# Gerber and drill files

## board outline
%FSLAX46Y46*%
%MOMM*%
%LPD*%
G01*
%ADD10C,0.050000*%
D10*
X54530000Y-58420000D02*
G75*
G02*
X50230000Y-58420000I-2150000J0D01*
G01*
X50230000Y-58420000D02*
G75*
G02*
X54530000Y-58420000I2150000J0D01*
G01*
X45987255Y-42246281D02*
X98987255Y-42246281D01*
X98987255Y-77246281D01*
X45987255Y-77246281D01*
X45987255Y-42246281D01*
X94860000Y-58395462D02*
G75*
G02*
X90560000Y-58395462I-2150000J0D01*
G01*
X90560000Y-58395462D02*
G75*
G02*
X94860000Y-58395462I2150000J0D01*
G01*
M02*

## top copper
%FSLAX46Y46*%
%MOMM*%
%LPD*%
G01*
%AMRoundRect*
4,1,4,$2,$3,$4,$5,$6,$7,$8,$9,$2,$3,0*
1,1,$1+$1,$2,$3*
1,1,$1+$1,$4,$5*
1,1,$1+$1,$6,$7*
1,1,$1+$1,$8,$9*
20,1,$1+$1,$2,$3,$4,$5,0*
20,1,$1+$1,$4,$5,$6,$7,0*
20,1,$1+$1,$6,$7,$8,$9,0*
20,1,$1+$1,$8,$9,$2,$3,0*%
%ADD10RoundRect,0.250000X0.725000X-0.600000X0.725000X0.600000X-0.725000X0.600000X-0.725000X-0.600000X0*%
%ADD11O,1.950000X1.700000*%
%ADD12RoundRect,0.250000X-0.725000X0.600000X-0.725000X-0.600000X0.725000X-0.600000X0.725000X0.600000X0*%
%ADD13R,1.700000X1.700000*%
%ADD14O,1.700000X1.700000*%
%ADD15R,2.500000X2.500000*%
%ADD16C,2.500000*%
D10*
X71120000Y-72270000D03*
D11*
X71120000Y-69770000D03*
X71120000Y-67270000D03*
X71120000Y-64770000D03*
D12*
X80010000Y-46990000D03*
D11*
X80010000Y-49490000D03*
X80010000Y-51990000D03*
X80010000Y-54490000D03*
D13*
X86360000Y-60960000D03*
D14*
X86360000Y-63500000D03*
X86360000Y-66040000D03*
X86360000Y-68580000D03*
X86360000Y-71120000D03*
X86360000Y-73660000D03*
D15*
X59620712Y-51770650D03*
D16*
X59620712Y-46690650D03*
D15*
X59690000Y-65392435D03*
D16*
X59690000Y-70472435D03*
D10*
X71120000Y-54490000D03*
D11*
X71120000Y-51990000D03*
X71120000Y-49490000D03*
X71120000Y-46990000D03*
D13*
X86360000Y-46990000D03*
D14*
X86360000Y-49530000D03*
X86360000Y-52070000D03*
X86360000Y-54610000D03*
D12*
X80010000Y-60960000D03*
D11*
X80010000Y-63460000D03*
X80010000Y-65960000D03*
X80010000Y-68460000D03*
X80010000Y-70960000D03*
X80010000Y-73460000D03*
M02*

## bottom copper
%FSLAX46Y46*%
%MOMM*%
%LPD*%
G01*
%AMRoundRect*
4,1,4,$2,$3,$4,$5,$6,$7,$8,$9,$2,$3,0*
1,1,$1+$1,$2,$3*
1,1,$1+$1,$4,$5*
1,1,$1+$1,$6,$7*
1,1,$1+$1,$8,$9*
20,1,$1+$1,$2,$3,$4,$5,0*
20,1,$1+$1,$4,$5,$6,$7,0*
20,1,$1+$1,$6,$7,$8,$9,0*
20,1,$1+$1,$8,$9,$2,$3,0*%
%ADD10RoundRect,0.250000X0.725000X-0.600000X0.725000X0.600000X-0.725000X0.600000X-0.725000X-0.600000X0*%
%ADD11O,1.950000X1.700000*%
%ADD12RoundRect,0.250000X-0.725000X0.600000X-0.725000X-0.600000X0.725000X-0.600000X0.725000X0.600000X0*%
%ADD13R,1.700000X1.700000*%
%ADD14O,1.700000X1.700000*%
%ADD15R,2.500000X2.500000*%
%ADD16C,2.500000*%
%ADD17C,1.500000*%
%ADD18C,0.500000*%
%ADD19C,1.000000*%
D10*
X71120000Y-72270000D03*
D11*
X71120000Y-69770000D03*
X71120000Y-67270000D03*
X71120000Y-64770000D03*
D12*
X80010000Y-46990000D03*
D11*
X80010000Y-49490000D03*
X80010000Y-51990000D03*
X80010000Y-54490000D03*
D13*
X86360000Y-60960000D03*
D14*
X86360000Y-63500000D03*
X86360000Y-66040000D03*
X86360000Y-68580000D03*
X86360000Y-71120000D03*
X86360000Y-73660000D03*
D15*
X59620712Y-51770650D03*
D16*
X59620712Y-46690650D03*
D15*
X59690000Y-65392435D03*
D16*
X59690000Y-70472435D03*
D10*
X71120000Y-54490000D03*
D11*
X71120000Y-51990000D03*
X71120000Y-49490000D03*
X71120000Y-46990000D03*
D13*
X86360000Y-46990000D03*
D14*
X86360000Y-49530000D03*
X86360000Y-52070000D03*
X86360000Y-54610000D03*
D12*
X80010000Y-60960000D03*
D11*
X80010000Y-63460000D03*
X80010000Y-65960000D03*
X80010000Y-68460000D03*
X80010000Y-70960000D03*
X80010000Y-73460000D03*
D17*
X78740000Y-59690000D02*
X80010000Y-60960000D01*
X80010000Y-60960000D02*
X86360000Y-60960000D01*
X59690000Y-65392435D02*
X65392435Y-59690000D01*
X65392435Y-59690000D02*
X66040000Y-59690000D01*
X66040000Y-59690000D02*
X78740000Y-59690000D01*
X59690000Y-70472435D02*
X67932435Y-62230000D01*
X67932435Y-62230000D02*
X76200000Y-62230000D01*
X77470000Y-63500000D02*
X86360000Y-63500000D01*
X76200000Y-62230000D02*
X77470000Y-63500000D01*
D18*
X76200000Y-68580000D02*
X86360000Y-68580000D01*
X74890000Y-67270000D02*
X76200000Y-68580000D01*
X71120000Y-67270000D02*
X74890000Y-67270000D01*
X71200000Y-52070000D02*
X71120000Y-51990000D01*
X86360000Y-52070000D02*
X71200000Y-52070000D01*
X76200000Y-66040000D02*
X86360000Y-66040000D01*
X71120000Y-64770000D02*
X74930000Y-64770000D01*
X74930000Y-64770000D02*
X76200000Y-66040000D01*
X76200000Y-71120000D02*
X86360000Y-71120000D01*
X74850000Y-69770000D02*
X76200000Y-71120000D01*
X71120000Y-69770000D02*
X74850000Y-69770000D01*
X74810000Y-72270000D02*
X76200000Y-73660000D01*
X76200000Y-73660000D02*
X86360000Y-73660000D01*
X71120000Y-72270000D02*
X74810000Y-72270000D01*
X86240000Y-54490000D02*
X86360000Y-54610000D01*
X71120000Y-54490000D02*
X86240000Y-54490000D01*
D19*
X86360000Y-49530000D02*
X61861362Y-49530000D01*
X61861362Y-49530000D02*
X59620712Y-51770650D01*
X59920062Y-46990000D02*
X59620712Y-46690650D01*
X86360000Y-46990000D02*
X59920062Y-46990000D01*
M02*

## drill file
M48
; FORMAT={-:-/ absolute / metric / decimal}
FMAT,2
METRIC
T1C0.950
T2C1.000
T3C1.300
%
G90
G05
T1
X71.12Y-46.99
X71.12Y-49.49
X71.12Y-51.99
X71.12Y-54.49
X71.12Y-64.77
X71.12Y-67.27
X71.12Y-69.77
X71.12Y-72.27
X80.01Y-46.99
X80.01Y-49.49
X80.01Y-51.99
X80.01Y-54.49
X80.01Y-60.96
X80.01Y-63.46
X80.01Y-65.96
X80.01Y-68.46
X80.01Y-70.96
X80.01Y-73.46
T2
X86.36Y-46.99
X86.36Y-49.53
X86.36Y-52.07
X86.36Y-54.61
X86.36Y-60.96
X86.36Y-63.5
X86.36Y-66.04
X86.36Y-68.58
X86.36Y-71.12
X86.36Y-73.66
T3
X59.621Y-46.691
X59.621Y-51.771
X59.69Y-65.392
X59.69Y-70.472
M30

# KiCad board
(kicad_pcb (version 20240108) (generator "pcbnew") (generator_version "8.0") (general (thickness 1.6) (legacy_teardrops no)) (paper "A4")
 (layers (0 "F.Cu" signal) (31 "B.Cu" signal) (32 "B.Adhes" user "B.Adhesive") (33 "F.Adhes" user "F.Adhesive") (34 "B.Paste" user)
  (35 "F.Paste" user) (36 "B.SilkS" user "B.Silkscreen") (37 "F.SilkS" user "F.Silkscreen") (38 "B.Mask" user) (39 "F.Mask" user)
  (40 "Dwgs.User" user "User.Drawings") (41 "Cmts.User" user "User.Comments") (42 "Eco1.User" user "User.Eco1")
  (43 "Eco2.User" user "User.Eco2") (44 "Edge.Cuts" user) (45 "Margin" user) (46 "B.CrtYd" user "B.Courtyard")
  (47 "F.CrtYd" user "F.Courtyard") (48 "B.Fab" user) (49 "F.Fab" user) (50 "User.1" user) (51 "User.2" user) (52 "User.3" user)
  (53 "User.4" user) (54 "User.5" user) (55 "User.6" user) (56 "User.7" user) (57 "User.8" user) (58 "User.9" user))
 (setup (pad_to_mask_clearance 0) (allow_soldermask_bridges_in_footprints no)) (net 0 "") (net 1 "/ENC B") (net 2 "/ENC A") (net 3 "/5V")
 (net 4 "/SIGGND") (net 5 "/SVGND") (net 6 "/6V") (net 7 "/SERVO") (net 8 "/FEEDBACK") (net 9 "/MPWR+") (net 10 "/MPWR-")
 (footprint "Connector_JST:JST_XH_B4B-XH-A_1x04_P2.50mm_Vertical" (layer "F.Cu") (at 71.12 72.27 90)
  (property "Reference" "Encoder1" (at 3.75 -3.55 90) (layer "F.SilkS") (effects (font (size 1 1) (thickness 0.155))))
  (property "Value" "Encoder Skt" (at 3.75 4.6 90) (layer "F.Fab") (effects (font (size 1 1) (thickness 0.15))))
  (pad "1" thru_hole roundrect (at 0 0 90) (size 1.7 1.95) (drill 0.95) (layers "*.Cu" "*.Mask") (remove_unused_layers no)
   (roundrect_rratio 0.147059) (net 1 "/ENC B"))
  (pad "2" thru_hole oval (at 2.5 0 90) (size 1.7 1.95) (drill 0.95) (layers "*.Cu" "*.Mask") (remove_unused_layers no) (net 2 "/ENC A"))
  (pad "3" thru_hole oval (at 5 0 90) (size 1.7 1.95) (drill 0.95) (layers "*.Cu" "*.Mask") (remove_unused_layers no) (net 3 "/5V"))
  (pad "4" thru_hole oval (at 7.5 0 90) (size 1.7 1.95) (drill 0.95) (layers "*.Cu" "*.Mask") (remove_unused_layers no) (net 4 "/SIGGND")))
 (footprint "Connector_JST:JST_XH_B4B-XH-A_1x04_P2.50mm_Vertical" (layer "F.Cu") (at 80.01 46.99 -90)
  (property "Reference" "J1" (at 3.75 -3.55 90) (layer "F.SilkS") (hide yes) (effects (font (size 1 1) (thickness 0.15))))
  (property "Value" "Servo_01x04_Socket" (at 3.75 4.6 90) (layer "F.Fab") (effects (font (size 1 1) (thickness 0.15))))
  (pad "1" thru_hole roundrect (at 0 0 270) (size 1.7 1.95) (drill 0.95) (layers "*.Cu" "*.Mask") (remove_unused_layers no)
   (roundrect_rratio 0.147059) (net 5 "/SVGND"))
  (pad "2" thru_hole oval (at 2.5 0 270) (size 1.7 1.95) (drill 0.95) (layers "*.Cu" "*.Mask") (remove_unused_layers no) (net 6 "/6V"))
  (pad "3" thru_hole oval (at 5 0 270) (size 1.7 1.95) (drill 0.95) (layers "*.Cu" "*.Mask") (remove_unused_layers no) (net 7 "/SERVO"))
  (pad "4" thru_hole oval (at 7.5 0 270) (size 1.7 1.95) (drill 0.95) (layers "*.Cu" "*.Mask") (remove_unused_layers no) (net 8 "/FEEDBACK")))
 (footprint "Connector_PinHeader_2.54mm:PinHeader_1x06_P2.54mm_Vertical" (layer "F.Cu") (at 86.36 60.96)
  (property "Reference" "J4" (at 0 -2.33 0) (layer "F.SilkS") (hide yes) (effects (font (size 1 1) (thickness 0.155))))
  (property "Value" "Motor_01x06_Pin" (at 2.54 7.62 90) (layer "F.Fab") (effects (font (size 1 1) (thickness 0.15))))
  (pad "1" thru_hole rect (at 0 0) (size 1.7 1.7) (drill 1) (layers "*.Cu" "*.Mask") (remove_unused_layers no) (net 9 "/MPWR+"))
  (pad "2" thru_hole oval (at 0 2.54) (size 1.7 1.7) (drill 1) (layers "*.Cu" "*.Mask") (remove_unused_layers no) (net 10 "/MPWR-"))
  (pad "3" thru_hole oval (at 0 5.08) (size 1.7 1.7) (drill 1) (layers "*.Cu" "*.Mask") (remove_unused_layers no) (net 4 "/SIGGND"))
  (pad "4" thru_hole oval (at 0 7.62) (size 1.7 1.7) (drill 1) (layers "*.Cu" "*.Mask") (remove_unused_layers no) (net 3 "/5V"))
  (pad "5" thru_hole oval (at 0 10.16) (size 1.7 1.7) (drill 1) (layers "*.Cu" "*.Mask") (remove_unused_layers no) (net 2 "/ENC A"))
  (pad "6" thru_hole oval (at 0 12.7) (size 1.7 1.7) (drill 1) (layers "*.Cu" "*.Mask") (remove_unused_layers no) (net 1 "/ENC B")))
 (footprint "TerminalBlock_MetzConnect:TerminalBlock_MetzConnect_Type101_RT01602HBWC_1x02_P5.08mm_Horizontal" (layer "F.Cu")
  (at 59.620712 51.77065 90)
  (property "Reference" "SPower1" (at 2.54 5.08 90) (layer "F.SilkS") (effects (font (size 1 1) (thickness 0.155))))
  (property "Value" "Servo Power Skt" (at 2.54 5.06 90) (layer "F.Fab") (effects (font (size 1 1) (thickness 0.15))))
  (pad "1" thru_hole rect (at 0 0 90) (size 2.5 2.5) (drill 1.3) (layers "*.Cu" "*.Mask") (remove_unused_layers no) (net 6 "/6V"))
  (pad "2" thru_hole circle (at 5.08 0 90) (size 2.5 2.5) (drill 1.3) (layers "*.Cu" "*.Mask") (remove_unused_layers no) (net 5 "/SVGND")))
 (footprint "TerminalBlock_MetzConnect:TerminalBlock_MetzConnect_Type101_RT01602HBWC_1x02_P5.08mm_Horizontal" (layer "F.Cu")
  (at 59.69 65.392435 -90)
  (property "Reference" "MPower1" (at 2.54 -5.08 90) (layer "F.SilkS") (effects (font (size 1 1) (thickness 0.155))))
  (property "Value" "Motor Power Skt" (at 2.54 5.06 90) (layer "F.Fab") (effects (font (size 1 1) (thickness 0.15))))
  (pad "1" thru_hole rect (at 0 0 270) (size 2.5 2.5) (drill 1.3) (layers "*.Cu" "*.Mask") (remove_unused_layers no) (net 9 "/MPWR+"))
  (pad "2" thru_hole circle (at 5.08 0 270) (size 2.5 2.5) (drill 1.3) (layers "*.Cu" "*.Mask") (remove_unused_layers no) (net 10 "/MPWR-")))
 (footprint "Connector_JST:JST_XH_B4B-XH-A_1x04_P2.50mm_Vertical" (layer "F.Cu") (at 71.12 54.49 90)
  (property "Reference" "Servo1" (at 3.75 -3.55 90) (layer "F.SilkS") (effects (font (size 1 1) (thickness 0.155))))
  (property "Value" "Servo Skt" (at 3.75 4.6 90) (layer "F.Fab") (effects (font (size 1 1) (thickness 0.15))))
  (pad "1" thru_hole roundrect (at 0 0 90) (size 1.7 1.95) (drill 0.95) (layers "*.Cu" "*.Mask") (remove_unused_layers no)
   (roundrect_rratio 0.147059) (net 8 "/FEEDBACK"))
  (pad "2" thru_hole oval (at 2.5 0 90) (size 1.7 1.95) (drill 0.95) (layers "*.Cu" "*.Mask") (remove_unused_layers no) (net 7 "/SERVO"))
  (pad "3" thru_hole oval (at 5 0 90) (size 1.7 1.95) (drill 0.95) (layers "*.Cu" "*.Mask") (remove_unused_layers no) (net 6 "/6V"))
  (pad "4" thru_hole oval (at 7.5 0 90) (size 1.7 1.95) (drill 0.95) (layers "*.Cu" "*.Mask") (remove_unused_layers no) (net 5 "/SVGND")))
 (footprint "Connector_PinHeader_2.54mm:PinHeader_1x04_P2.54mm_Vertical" (layer "F.Cu") (at 86.36 46.99)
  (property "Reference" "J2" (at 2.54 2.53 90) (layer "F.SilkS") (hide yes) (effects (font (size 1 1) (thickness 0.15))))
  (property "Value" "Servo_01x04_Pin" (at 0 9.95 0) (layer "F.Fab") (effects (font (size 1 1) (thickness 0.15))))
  (pad "1" thru_hole rect (at 0 0) (size 1.7 1.7) (drill 1) (layers "*.Cu" "*.Mask") (remove_unused_layers no) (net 5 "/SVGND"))
  (pad "2" thru_hole oval (at 0 2.54) (size 1.7 1.7) (drill 1) (layers "*.Cu" "*.Mask") (remove_unused_layers no) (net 6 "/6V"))
  (pad "3" thru_hole oval (at 0 5.08) (size 1.7 1.7) (drill 1) (layers "*.Cu" "*.Mask") (remove_unused_layers no) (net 7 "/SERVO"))
  (pad "4" thru_hole oval (at 0 7.62) (size 1.7 1.7) (drill 1) (layers "*.Cu" "*.Mask") (remove_unused_layers no) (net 8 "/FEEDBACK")))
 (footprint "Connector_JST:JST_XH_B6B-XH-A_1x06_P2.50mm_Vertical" (layer "F.Cu") (at 80.01 60.96 -90)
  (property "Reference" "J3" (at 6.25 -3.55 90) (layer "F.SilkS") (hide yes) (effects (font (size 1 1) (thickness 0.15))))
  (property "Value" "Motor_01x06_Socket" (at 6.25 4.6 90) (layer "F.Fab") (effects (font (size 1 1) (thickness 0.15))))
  (pad "1" thru_hole roundrect (at 0 0 270) (size 1.7 1.95) (drill 0.95) (layers "*.Cu" "*.Mask") (remove_unused_layers no)
   (roundrect_rratio 0.147059) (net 9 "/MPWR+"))
  (pad "2" thru_hole oval (at 2.5 0 270) (size 1.7 1.95) (drill 0.95) (layers "*.Cu" "*.Mask") (remove_unused_layers no) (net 10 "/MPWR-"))
  (pad "3" thru_hole oval (at 5 0 270) (size 1.7 1.95) (drill 0.95) (layers "*.Cu" "*.Mask") (remove_unused_layers no) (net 4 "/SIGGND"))
  (pad "4" thru_hole oval (at 7.5 0 270) (size 1.7 1.95) (drill 0.95) (layers "*.Cu" "*.Mask") (remove_unused_layers no) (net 3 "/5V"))
  (pad "5" thru_hole oval (at 10 0 270) (size 1.7 1.95) (drill 0.95) (layers "*.Cu" "*.Mask") (remove_unused_layers no) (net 2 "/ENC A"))
  (pad "6" thru_hole oval (at 12.5 0 270) (size 1.7 1.95) (drill 0.95) (layers "*.Cu" "*.Mask") (remove_unused_layers no) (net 1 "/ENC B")))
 (gr_circle (center 52.38 58.42) (end 54.53 58.42) (stroke (width 0.05) (type default)) (fill none) (layer "Edge.Cuts"))
 (gr_rect (start 45.987255 42.246281) (end 98.987255 77.246281) (stroke (width 0.05) (type default)) (fill none) (layer "Edge.Cuts"))
 (gr_circle (center 92.71 58.395462) (end 94.86 58.395462) (stroke (width 0.05) (type default)) (fill none) (layer "Edge.Cuts"))
 (segment (start 78.74 59.69) (end 80.01 60.96) (width 1.5) (layer "B.Cu") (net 9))
 (segment (start 80.01 60.96) (end 86.36 60.96) (width 1.5) (layer "B.Cu") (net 9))
 (segment (start 59.69 65.392435) (end 65.392435 59.69) (width 1.5) (layer "B.Cu") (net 9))
 (segment (start 65.392435 59.69) (end 66.04 59.69) (width 1.5) (layer "B.Cu") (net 9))
 (segment (start 66.04 59.69) (end 78.74 59.69) (width 1.5) (layer "B.Cu") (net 9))
 (segment (start 59.69 70.472435) (end 67.932435 62.23) (width 1.5) (layer "B.Cu") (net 10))
 (segment (start 67.932435 62.23) (end 76.2 62.23) (width 1.5) (layer "B.Cu") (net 10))
 (segment (start 77.47 63.5) (end 86.36 63.5) (width 1.5) (layer "B.Cu") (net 10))
 (segment (start 76.2 62.23) (end 77.47 63.5) (width 1.5) (layer "B.Cu") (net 10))
 (segment (start 76.2 68.58) (end 86.36 68.58) (width 0.5) (layer "B.Cu") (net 3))
 (segment (start 74.89 67.27) (end 76.2 68.58) (width 0.5) (layer "B.Cu") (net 3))
 (segment (start 71.12 67.27) (end 74.89 67.27) (width 0.5) (layer "B.Cu") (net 3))
 (segment (start 71.2 52.07) (end 71.12 51.99) (width 0.5) (layer "B.Cu") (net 7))
 (segment (start 86.36 52.07) (end 71.2 52.07) (width 0.5) (layer "B.Cu") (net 7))
 (segment (start 76.2 66.04) (end 86.36 66.04) (width 0.5) (layer "B.Cu") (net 4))
 (segment (start 71.12 64.77) (end 74.93 64.77) (width 0.5) (layer "B.Cu") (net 4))
 (segment (start 74.93 64.77) (end 76.2 66.04) (width 0.5) (layer "B.Cu") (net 4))
 (segment (start 76.2 71.12) (end 86.36 71.12) (width 0.5) (layer "B.Cu") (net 2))
 (segment (start 74.85 69.77) (end 76.2 71.12) (width 0.5) (layer "B.Cu") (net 2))
 (segment (start 71.12 69.77) (end 74.85 69.77) (width 0.5) (layer "B.Cu") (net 2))
 (segment (start 74.81 72.27) (end 76.2 73.66) (width 0.5) (layer "B.Cu") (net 1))
 (segment (start 76.2 73.66) (end 86.36 73.66) (width 0.5) (layer "B.Cu") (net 1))
 (segment (start 71.12 72.27) (end 74.81 72.27) (width 0.5) (layer "B.Cu") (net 1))
 (segment (start 86.24 54.49) (end 86.36 54.61) (width 0.5) (layer "B.Cu") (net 8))
 (segment (start 71.12 54.49) (end 86.24 54.49) (width 0.5) (layer "B.Cu") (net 8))
 (segment (start 86.36 49.53) (end 61.861362 49.53) (width 1) (layer "B.Cu") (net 6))
 (segment (start 61.861362 49.53) (end 59.620712 51.77065) (width 1) (layer "B.Cu") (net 6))
 (segment (start 59.920062 46.99) (end 59.620712 46.69065) (width 1) (layer "B.Cu") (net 5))
 (segment (start 86.36 46.99) (end 59.920062 46.99) (width 1) (layer "B.Cu") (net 5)))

